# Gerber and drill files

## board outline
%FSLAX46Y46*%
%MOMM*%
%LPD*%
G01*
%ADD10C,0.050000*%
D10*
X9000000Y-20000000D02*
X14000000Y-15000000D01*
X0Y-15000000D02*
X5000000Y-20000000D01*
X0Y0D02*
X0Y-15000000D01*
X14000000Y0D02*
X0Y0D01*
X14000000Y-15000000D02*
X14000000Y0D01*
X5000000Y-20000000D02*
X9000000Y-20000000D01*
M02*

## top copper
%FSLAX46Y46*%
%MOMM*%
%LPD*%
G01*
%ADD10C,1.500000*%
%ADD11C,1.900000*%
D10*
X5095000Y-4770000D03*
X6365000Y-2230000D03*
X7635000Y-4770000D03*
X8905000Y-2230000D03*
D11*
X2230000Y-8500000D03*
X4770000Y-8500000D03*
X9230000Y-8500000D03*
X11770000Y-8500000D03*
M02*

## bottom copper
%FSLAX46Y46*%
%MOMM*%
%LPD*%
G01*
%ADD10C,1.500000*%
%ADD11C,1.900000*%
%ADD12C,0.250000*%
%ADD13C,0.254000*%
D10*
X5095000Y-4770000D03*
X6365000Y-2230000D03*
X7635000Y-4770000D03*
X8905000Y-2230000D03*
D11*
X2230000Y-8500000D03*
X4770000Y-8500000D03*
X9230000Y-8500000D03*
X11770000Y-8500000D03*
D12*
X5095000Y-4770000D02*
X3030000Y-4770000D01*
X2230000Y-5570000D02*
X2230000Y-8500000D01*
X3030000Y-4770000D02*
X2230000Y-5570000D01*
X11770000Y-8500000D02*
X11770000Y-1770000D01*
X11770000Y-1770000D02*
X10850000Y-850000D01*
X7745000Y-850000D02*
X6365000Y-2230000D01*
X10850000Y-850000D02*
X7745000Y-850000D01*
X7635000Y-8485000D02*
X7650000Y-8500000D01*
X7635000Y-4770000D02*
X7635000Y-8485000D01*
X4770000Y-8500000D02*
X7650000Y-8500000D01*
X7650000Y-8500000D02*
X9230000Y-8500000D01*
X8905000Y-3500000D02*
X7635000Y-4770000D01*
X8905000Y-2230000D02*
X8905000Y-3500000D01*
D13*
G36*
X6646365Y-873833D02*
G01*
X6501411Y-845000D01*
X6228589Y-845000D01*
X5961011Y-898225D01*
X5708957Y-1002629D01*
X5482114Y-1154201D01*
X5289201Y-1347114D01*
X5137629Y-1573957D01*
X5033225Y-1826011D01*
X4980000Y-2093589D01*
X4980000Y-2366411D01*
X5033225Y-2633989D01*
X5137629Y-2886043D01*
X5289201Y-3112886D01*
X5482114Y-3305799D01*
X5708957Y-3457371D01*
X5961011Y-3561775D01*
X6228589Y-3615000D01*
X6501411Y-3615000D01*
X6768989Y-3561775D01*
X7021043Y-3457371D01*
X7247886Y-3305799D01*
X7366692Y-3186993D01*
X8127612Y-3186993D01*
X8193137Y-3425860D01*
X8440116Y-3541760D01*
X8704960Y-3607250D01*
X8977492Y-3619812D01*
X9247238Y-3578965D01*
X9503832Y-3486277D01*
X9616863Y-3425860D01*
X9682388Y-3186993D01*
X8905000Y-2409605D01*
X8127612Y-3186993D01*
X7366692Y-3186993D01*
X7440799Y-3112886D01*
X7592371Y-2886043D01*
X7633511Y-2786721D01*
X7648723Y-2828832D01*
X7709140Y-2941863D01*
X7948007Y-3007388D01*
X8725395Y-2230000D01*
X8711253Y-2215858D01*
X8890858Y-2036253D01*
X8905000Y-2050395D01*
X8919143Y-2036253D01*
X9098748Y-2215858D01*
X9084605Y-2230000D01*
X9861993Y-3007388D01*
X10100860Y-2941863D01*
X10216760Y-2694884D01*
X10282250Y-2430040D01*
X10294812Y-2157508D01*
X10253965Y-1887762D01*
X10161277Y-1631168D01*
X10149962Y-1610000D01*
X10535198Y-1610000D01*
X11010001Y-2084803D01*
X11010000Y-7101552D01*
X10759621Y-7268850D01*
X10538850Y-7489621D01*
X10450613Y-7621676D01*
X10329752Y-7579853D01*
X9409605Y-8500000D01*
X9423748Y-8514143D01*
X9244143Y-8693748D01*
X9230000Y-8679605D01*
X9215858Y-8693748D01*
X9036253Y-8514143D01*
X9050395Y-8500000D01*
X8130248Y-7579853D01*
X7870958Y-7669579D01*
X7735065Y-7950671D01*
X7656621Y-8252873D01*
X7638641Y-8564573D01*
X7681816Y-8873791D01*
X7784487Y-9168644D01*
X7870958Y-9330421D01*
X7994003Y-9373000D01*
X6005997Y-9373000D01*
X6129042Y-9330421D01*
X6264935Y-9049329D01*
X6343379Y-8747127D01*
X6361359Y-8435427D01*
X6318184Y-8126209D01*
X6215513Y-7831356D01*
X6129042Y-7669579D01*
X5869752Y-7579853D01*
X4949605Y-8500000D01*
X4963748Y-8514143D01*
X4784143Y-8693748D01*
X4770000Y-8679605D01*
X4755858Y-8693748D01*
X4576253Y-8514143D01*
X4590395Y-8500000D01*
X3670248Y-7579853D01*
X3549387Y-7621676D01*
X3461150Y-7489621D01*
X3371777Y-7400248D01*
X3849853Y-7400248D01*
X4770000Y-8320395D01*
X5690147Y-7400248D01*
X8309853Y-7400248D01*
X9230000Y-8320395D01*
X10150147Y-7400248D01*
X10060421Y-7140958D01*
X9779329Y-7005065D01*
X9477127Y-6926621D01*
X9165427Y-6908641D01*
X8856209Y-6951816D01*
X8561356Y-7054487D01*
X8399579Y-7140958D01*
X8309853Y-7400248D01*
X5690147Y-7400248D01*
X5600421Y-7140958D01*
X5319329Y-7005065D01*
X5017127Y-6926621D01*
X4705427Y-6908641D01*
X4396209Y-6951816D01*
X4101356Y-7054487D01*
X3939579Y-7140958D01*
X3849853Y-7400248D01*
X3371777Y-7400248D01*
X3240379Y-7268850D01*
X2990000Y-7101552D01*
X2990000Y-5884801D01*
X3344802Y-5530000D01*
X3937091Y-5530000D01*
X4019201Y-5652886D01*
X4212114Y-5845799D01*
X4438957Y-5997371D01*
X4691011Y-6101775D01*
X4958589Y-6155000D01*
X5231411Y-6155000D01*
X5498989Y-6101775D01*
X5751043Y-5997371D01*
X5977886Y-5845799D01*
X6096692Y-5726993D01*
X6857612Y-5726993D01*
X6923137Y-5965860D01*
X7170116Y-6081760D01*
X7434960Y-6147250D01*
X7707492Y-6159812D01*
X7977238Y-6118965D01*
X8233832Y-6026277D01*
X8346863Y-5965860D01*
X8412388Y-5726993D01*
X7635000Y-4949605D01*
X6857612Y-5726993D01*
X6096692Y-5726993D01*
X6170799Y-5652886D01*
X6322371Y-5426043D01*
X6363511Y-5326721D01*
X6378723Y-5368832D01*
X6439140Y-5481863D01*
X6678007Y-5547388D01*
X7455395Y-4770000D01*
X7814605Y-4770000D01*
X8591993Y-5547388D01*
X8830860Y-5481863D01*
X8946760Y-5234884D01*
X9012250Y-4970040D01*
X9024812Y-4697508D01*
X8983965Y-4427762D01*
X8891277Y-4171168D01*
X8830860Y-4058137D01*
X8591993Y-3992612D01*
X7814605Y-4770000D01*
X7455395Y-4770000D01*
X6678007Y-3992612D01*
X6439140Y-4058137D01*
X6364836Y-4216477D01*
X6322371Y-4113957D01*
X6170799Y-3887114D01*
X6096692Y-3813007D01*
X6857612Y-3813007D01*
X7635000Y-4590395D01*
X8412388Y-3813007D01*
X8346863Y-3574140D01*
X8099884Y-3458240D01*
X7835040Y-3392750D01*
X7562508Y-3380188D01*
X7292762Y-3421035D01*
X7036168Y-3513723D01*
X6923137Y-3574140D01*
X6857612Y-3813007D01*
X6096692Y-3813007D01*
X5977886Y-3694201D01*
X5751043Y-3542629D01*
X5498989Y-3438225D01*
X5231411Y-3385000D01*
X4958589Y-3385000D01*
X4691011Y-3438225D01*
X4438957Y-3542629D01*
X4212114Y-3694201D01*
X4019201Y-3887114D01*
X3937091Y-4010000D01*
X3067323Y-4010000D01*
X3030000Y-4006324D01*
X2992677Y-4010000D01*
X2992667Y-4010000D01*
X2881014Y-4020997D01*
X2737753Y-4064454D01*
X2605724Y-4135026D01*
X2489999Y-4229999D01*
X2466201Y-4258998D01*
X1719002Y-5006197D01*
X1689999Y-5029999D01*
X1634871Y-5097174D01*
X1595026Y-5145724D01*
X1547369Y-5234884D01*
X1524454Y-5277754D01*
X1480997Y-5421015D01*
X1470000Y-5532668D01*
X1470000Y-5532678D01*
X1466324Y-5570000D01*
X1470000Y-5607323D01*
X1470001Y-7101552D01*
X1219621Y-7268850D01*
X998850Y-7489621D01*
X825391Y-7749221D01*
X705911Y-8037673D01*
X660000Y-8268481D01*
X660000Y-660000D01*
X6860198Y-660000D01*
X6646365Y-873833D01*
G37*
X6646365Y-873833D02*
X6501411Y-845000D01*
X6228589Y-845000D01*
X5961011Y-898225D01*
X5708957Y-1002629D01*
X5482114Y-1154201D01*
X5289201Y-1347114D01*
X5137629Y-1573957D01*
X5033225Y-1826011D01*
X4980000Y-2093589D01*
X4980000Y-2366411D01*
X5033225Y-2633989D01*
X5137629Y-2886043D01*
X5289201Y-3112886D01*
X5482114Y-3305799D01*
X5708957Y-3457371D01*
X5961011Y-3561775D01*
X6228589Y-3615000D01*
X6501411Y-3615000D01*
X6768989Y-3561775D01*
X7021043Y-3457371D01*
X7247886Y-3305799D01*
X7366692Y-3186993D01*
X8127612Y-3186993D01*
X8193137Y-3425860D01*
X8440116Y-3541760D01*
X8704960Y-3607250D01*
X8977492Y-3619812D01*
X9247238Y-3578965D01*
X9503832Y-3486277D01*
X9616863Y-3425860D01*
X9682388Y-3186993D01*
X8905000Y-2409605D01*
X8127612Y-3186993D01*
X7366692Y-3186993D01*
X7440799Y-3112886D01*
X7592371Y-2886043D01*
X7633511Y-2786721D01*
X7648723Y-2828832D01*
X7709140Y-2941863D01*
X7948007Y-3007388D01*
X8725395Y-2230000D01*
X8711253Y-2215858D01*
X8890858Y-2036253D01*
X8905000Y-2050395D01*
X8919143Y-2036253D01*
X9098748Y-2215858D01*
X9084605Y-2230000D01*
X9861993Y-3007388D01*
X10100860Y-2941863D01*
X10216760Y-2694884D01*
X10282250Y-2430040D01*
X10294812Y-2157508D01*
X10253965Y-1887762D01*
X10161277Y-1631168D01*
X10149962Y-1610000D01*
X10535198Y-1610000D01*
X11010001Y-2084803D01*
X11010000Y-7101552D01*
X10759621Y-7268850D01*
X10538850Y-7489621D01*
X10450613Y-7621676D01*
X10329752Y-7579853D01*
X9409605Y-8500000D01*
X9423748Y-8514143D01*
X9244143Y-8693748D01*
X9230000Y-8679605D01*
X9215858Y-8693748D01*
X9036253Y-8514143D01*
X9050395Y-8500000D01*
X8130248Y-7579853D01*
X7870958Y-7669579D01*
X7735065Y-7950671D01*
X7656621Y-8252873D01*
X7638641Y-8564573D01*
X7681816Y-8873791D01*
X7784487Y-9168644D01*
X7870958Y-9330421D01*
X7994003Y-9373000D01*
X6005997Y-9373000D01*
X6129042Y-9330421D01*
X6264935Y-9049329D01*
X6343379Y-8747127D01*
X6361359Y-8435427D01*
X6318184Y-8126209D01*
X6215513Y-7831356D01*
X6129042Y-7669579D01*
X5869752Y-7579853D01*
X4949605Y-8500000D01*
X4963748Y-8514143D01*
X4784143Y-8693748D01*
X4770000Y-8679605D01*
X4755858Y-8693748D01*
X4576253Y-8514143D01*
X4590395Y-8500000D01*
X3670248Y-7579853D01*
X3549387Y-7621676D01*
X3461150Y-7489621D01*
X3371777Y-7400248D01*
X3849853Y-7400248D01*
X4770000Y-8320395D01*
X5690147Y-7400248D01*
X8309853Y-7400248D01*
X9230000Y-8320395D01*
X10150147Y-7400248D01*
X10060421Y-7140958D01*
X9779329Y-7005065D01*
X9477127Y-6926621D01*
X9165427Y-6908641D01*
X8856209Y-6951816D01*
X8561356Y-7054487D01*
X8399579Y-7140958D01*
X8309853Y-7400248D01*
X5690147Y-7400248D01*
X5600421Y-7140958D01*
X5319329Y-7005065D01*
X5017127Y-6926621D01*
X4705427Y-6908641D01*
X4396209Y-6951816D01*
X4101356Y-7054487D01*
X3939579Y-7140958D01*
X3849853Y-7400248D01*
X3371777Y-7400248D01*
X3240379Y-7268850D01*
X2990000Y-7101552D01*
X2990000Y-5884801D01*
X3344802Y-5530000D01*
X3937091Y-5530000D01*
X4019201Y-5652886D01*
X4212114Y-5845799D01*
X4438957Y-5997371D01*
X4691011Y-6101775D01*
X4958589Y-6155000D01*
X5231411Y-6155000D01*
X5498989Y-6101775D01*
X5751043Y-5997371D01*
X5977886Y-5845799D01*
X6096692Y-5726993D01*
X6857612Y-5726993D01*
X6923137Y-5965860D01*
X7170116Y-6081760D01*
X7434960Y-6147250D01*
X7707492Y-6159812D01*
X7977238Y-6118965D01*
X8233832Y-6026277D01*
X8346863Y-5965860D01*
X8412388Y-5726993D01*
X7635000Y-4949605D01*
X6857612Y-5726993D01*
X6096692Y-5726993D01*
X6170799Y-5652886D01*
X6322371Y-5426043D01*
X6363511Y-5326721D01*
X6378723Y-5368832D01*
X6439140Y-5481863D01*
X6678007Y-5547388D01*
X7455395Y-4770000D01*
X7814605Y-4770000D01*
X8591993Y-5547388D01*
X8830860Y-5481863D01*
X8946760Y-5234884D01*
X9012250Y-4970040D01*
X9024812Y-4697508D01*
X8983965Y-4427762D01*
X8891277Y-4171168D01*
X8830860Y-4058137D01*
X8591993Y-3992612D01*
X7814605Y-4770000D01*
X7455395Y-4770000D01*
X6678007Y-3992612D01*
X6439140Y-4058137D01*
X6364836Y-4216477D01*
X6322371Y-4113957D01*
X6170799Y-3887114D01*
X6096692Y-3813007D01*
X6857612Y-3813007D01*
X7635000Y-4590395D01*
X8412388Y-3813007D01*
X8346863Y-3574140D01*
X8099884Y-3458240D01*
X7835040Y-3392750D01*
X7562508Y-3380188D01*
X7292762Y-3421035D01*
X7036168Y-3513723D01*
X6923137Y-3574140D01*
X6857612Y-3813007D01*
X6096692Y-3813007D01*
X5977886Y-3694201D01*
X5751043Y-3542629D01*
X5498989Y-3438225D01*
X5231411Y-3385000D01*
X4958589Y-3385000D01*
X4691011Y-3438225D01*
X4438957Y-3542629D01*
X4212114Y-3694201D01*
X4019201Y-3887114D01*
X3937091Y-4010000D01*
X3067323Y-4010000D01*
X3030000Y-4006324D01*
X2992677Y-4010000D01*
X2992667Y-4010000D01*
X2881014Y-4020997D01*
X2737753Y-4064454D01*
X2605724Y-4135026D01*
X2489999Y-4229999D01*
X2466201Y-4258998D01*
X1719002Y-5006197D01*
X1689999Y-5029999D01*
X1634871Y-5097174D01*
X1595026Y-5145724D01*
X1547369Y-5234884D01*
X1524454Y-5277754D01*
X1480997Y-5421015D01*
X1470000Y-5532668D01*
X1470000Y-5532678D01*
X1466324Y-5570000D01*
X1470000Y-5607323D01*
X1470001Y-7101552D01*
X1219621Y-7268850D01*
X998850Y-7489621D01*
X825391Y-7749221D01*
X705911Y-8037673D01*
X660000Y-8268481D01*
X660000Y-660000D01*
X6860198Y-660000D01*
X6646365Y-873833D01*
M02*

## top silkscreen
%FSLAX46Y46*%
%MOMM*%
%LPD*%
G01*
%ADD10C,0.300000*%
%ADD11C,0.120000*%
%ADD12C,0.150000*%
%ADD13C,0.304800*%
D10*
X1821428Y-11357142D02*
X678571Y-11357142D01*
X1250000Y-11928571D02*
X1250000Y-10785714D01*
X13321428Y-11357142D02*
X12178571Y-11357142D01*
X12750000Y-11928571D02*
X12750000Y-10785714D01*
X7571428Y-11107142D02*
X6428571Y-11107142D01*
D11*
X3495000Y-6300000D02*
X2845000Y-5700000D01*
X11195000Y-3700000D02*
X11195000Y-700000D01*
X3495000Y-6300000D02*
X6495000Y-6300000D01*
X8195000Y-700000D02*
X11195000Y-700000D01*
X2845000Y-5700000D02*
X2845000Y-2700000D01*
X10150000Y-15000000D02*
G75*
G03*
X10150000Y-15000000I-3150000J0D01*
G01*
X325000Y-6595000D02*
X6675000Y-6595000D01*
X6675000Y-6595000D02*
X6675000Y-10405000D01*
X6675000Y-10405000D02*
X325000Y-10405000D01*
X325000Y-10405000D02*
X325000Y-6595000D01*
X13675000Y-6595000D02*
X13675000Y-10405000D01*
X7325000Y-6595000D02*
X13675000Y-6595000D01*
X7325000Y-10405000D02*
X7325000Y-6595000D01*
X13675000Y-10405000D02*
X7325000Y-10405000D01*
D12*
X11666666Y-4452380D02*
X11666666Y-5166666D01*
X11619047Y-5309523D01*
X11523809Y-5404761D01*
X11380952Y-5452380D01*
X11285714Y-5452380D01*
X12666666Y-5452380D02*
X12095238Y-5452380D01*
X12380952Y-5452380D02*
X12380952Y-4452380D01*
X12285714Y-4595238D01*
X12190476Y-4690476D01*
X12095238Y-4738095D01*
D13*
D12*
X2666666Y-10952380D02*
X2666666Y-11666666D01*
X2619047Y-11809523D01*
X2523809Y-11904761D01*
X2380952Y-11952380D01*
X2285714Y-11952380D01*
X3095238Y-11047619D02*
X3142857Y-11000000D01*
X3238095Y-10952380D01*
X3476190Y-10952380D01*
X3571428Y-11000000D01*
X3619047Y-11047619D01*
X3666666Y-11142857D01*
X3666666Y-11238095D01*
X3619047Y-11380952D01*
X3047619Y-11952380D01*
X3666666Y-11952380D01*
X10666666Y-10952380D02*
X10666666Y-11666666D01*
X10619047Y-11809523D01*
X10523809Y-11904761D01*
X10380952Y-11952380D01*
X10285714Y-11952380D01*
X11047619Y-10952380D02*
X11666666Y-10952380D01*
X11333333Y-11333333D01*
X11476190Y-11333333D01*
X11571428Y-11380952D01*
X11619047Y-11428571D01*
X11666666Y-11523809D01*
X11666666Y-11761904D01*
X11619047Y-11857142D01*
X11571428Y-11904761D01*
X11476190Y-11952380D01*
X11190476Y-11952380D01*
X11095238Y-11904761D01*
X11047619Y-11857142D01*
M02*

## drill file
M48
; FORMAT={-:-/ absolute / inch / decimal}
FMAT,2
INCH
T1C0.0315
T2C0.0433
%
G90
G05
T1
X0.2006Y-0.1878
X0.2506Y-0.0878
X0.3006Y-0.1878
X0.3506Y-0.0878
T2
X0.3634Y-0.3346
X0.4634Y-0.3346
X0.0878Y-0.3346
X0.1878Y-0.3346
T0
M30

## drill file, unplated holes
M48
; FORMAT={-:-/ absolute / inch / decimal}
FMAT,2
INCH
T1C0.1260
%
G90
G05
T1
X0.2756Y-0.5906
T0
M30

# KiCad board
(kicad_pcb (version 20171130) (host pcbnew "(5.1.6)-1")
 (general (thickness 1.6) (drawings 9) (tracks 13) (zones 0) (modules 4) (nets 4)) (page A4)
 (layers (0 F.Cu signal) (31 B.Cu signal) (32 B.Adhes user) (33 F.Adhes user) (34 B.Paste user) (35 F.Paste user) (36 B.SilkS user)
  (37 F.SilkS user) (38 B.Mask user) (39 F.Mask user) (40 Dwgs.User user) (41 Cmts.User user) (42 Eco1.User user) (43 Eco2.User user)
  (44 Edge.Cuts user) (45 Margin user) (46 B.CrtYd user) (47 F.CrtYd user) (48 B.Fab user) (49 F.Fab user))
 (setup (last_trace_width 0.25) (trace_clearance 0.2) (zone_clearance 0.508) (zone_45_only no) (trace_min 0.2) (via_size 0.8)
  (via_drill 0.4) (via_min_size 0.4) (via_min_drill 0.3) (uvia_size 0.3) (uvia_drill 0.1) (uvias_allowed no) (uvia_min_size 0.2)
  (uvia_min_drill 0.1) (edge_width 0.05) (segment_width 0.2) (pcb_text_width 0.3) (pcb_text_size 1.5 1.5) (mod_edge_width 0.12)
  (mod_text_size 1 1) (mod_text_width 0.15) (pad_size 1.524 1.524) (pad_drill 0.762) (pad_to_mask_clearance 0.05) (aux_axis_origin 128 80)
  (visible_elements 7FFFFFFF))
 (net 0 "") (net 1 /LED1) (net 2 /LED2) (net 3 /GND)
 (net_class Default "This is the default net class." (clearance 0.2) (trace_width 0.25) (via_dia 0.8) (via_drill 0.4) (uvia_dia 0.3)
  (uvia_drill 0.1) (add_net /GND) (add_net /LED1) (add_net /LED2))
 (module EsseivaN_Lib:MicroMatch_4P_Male (layer F.Cu) (at 135 83.5)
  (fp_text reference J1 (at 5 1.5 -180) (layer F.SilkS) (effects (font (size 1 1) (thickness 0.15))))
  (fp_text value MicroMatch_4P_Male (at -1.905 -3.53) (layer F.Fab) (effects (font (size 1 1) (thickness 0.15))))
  (fp_line (start -3.505 2.8) (end -4.155 2.2) (layer F.SilkS) (width 0.12))
  (fp_line (start 4.195 0.2) (end 4.195 -2.8) (layer F.SilkS) (width 0.12))
  (fp_line (start -3.505 2.8) (end -0.505 2.8) (layer F.SilkS) (width 0.12))
  (fp_line (start 1.195 -2.8) (end 4.195 -2.8) (layer F.SilkS) (width 0.12))
  (fp_line (start -4.155 2.2) (end -4.155 -0.8) (layer F.SilkS) (width 0.12))
  (pad 1 thru_hole circle (at -1.905 1.27 90) (size 1.5 1.5) (drill 0.8) (layers *.Cu *.Mask) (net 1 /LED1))
  (pad 2 thru_hole circle (at -0.635 -1.27 90) (size 1.5 1.5) (drill 0.8) (layers *.Cu *.Mask) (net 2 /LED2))
  (pad 3 thru_hole circle (at 0.635 1.27 90) (size 1.5 1.5) (drill 0.8) (layers *.Cu *.Mask) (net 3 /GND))
  (pad 4 thru_hole circle (at 1.905 -1.27 90) (size 1.5 1.5) (drill 0.8) (layers *.Cu *.Mask) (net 3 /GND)))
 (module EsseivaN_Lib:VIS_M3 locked (layer F.Cu) (at 135 95)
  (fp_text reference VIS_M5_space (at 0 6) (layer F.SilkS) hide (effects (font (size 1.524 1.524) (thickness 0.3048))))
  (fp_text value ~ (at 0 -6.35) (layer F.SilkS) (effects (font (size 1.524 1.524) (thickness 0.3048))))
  (fp_circle (center 0 0) (end 3.15 0) (layer F.SilkS) (width 0.12))
  (pad "" np_thru_hole circle (at 0 0) (size 3.2 3.2) (drill 3.2) (layers *.Cu *.Mask)))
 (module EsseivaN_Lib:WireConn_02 (layer F.Cu) (at 131.5 88.5)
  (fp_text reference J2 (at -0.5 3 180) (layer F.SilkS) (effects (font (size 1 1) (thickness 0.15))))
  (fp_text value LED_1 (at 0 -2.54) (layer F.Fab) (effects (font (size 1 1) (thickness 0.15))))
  (fp_line (start -3.175 -1.905) (end 3.175 -1.905) (layer F.SilkS) (width 0.12))
  (fp_line (start 3.175 -1.905) (end 3.175 1.905) (layer F.SilkS) (width 0.12))
  (fp_line (start 3.175 1.905) (end -3.175 1.905) (layer F.SilkS) (width 0.12))
  (fp_line (start -3.175 1.905) (end -3.175 -1.905) (layer F.SilkS) (width 0.12))
  (pad 1 thru_hole circle (at -1.27 0) (size 1.9 1.9) (drill 1.1) (layers *.Cu *.Mask) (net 1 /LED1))
  (pad 2 thru_hole circle (at 1.27 0) (size 1.9 1.9) (drill 1.1) (layers *.Cu *.Mask) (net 3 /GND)))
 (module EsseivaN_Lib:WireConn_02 (layer F.Cu) (at 138.5 88.5 180)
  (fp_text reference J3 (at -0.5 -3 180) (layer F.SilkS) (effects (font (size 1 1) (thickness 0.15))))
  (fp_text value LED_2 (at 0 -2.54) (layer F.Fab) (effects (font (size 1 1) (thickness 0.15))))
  (fp_line (start -3.175 1.905) (end -3.175 -1.905) (layer F.SilkS) (width 0.12))
  (fp_line (start 3.175 1.905) (end -3.175 1.905) (layer F.SilkS) (width 0.12))
  (fp_line (start 3.175 -1.905) (end 3.175 1.905) (layer F.SilkS) (width 0.12))
  (fp_line (start -3.175 -1.905) (end 3.175 -1.905) (layer F.SilkS) (width 0.12))
  (pad 2 thru_hole circle (at 1.27 0 180) (size 1.9 1.9) (drill 1.1) (layers *.Cu *.Mask) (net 3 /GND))
  (pad 1 thru_hole circle (at -1.27 0 180) (size 1.9 1.9) (drill 1.1) (layers *.Cu *.Mask) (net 2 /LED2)))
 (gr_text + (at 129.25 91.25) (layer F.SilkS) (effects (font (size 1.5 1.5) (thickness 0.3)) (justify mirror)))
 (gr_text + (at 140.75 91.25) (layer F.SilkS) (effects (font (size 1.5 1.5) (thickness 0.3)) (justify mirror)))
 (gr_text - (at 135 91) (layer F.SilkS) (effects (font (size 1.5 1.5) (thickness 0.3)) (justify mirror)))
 (gr_line (start 137 100) (end 142 95) (layer Edge.Cuts) (width 0.05))
 (gr_line (start 128 95) (end 133 100) (layer Edge.Cuts) (width 0.05))
 (gr_line (start 128 80) (end 128 95) (layer Edge.Cuts) (width 0.05))
 (gr_line (start 142 80) (end 128 80) (layer Edge.Cuts) (width 0.05))
 (gr_line (start 142 95) (end 142 80) (layer Edge.Cuts) (width 0.05))
 (gr_line (start 133 100) (end 137 100) (layer Edge.Cuts) (width 0.05))
 (segment (start 133.095 84.77) (end 131.03 84.77) (width 0.25) (layer B.Cu) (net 1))
 (segment (start 130.23 85.57) (end 130.23 88.5) (width 0.25) (layer B.Cu) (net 1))
 (segment (start 131.03 84.77) (end 130.23 85.57) (width 0.25) (layer B.Cu) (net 1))
 (segment (start 139.77 88.5) (end 139.77 81.77) (width 0.25) (layer B.Cu) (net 2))
 (segment (start 139.77 81.77) (end 138.85 80.85) (width 0.25) (layer B.Cu) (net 2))
 (segment (start 135.745 80.85) (end 134.365 82.23) (width 0.25) (layer B.Cu) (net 2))
 (segment (start 138.85 80.85) (end 135.745 80.85) (width 0.25) (layer B.Cu) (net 2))
 (segment (start 135.635 88.485) (end 135.65 88.5) (width 0.25) (layer B.Cu) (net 3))
 (segment (start 135.635 84.77) (end 135.635 88.485) (width 0.25) (layer B.Cu) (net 3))
 (segment (start 132.77 88.5) (end 135.65 88.5) (width 0.25) (layer B.Cu) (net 3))
 (segment (start 135.65 88.5) (end 137.23 88.5) (width 0.25) (layer B.Cu) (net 3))
 (segment (start 136.905 83.5) (end 135.635 84.77) (width 0.25) (layer B.Cu) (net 3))
 (segment (start 136.905 82.23) (end 136.905 83.5) (width 0.25) (layer B.Cu) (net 3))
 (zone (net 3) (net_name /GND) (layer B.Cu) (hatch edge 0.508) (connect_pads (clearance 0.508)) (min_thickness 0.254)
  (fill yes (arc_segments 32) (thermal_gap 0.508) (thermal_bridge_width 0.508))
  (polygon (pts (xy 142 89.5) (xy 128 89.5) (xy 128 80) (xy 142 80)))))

